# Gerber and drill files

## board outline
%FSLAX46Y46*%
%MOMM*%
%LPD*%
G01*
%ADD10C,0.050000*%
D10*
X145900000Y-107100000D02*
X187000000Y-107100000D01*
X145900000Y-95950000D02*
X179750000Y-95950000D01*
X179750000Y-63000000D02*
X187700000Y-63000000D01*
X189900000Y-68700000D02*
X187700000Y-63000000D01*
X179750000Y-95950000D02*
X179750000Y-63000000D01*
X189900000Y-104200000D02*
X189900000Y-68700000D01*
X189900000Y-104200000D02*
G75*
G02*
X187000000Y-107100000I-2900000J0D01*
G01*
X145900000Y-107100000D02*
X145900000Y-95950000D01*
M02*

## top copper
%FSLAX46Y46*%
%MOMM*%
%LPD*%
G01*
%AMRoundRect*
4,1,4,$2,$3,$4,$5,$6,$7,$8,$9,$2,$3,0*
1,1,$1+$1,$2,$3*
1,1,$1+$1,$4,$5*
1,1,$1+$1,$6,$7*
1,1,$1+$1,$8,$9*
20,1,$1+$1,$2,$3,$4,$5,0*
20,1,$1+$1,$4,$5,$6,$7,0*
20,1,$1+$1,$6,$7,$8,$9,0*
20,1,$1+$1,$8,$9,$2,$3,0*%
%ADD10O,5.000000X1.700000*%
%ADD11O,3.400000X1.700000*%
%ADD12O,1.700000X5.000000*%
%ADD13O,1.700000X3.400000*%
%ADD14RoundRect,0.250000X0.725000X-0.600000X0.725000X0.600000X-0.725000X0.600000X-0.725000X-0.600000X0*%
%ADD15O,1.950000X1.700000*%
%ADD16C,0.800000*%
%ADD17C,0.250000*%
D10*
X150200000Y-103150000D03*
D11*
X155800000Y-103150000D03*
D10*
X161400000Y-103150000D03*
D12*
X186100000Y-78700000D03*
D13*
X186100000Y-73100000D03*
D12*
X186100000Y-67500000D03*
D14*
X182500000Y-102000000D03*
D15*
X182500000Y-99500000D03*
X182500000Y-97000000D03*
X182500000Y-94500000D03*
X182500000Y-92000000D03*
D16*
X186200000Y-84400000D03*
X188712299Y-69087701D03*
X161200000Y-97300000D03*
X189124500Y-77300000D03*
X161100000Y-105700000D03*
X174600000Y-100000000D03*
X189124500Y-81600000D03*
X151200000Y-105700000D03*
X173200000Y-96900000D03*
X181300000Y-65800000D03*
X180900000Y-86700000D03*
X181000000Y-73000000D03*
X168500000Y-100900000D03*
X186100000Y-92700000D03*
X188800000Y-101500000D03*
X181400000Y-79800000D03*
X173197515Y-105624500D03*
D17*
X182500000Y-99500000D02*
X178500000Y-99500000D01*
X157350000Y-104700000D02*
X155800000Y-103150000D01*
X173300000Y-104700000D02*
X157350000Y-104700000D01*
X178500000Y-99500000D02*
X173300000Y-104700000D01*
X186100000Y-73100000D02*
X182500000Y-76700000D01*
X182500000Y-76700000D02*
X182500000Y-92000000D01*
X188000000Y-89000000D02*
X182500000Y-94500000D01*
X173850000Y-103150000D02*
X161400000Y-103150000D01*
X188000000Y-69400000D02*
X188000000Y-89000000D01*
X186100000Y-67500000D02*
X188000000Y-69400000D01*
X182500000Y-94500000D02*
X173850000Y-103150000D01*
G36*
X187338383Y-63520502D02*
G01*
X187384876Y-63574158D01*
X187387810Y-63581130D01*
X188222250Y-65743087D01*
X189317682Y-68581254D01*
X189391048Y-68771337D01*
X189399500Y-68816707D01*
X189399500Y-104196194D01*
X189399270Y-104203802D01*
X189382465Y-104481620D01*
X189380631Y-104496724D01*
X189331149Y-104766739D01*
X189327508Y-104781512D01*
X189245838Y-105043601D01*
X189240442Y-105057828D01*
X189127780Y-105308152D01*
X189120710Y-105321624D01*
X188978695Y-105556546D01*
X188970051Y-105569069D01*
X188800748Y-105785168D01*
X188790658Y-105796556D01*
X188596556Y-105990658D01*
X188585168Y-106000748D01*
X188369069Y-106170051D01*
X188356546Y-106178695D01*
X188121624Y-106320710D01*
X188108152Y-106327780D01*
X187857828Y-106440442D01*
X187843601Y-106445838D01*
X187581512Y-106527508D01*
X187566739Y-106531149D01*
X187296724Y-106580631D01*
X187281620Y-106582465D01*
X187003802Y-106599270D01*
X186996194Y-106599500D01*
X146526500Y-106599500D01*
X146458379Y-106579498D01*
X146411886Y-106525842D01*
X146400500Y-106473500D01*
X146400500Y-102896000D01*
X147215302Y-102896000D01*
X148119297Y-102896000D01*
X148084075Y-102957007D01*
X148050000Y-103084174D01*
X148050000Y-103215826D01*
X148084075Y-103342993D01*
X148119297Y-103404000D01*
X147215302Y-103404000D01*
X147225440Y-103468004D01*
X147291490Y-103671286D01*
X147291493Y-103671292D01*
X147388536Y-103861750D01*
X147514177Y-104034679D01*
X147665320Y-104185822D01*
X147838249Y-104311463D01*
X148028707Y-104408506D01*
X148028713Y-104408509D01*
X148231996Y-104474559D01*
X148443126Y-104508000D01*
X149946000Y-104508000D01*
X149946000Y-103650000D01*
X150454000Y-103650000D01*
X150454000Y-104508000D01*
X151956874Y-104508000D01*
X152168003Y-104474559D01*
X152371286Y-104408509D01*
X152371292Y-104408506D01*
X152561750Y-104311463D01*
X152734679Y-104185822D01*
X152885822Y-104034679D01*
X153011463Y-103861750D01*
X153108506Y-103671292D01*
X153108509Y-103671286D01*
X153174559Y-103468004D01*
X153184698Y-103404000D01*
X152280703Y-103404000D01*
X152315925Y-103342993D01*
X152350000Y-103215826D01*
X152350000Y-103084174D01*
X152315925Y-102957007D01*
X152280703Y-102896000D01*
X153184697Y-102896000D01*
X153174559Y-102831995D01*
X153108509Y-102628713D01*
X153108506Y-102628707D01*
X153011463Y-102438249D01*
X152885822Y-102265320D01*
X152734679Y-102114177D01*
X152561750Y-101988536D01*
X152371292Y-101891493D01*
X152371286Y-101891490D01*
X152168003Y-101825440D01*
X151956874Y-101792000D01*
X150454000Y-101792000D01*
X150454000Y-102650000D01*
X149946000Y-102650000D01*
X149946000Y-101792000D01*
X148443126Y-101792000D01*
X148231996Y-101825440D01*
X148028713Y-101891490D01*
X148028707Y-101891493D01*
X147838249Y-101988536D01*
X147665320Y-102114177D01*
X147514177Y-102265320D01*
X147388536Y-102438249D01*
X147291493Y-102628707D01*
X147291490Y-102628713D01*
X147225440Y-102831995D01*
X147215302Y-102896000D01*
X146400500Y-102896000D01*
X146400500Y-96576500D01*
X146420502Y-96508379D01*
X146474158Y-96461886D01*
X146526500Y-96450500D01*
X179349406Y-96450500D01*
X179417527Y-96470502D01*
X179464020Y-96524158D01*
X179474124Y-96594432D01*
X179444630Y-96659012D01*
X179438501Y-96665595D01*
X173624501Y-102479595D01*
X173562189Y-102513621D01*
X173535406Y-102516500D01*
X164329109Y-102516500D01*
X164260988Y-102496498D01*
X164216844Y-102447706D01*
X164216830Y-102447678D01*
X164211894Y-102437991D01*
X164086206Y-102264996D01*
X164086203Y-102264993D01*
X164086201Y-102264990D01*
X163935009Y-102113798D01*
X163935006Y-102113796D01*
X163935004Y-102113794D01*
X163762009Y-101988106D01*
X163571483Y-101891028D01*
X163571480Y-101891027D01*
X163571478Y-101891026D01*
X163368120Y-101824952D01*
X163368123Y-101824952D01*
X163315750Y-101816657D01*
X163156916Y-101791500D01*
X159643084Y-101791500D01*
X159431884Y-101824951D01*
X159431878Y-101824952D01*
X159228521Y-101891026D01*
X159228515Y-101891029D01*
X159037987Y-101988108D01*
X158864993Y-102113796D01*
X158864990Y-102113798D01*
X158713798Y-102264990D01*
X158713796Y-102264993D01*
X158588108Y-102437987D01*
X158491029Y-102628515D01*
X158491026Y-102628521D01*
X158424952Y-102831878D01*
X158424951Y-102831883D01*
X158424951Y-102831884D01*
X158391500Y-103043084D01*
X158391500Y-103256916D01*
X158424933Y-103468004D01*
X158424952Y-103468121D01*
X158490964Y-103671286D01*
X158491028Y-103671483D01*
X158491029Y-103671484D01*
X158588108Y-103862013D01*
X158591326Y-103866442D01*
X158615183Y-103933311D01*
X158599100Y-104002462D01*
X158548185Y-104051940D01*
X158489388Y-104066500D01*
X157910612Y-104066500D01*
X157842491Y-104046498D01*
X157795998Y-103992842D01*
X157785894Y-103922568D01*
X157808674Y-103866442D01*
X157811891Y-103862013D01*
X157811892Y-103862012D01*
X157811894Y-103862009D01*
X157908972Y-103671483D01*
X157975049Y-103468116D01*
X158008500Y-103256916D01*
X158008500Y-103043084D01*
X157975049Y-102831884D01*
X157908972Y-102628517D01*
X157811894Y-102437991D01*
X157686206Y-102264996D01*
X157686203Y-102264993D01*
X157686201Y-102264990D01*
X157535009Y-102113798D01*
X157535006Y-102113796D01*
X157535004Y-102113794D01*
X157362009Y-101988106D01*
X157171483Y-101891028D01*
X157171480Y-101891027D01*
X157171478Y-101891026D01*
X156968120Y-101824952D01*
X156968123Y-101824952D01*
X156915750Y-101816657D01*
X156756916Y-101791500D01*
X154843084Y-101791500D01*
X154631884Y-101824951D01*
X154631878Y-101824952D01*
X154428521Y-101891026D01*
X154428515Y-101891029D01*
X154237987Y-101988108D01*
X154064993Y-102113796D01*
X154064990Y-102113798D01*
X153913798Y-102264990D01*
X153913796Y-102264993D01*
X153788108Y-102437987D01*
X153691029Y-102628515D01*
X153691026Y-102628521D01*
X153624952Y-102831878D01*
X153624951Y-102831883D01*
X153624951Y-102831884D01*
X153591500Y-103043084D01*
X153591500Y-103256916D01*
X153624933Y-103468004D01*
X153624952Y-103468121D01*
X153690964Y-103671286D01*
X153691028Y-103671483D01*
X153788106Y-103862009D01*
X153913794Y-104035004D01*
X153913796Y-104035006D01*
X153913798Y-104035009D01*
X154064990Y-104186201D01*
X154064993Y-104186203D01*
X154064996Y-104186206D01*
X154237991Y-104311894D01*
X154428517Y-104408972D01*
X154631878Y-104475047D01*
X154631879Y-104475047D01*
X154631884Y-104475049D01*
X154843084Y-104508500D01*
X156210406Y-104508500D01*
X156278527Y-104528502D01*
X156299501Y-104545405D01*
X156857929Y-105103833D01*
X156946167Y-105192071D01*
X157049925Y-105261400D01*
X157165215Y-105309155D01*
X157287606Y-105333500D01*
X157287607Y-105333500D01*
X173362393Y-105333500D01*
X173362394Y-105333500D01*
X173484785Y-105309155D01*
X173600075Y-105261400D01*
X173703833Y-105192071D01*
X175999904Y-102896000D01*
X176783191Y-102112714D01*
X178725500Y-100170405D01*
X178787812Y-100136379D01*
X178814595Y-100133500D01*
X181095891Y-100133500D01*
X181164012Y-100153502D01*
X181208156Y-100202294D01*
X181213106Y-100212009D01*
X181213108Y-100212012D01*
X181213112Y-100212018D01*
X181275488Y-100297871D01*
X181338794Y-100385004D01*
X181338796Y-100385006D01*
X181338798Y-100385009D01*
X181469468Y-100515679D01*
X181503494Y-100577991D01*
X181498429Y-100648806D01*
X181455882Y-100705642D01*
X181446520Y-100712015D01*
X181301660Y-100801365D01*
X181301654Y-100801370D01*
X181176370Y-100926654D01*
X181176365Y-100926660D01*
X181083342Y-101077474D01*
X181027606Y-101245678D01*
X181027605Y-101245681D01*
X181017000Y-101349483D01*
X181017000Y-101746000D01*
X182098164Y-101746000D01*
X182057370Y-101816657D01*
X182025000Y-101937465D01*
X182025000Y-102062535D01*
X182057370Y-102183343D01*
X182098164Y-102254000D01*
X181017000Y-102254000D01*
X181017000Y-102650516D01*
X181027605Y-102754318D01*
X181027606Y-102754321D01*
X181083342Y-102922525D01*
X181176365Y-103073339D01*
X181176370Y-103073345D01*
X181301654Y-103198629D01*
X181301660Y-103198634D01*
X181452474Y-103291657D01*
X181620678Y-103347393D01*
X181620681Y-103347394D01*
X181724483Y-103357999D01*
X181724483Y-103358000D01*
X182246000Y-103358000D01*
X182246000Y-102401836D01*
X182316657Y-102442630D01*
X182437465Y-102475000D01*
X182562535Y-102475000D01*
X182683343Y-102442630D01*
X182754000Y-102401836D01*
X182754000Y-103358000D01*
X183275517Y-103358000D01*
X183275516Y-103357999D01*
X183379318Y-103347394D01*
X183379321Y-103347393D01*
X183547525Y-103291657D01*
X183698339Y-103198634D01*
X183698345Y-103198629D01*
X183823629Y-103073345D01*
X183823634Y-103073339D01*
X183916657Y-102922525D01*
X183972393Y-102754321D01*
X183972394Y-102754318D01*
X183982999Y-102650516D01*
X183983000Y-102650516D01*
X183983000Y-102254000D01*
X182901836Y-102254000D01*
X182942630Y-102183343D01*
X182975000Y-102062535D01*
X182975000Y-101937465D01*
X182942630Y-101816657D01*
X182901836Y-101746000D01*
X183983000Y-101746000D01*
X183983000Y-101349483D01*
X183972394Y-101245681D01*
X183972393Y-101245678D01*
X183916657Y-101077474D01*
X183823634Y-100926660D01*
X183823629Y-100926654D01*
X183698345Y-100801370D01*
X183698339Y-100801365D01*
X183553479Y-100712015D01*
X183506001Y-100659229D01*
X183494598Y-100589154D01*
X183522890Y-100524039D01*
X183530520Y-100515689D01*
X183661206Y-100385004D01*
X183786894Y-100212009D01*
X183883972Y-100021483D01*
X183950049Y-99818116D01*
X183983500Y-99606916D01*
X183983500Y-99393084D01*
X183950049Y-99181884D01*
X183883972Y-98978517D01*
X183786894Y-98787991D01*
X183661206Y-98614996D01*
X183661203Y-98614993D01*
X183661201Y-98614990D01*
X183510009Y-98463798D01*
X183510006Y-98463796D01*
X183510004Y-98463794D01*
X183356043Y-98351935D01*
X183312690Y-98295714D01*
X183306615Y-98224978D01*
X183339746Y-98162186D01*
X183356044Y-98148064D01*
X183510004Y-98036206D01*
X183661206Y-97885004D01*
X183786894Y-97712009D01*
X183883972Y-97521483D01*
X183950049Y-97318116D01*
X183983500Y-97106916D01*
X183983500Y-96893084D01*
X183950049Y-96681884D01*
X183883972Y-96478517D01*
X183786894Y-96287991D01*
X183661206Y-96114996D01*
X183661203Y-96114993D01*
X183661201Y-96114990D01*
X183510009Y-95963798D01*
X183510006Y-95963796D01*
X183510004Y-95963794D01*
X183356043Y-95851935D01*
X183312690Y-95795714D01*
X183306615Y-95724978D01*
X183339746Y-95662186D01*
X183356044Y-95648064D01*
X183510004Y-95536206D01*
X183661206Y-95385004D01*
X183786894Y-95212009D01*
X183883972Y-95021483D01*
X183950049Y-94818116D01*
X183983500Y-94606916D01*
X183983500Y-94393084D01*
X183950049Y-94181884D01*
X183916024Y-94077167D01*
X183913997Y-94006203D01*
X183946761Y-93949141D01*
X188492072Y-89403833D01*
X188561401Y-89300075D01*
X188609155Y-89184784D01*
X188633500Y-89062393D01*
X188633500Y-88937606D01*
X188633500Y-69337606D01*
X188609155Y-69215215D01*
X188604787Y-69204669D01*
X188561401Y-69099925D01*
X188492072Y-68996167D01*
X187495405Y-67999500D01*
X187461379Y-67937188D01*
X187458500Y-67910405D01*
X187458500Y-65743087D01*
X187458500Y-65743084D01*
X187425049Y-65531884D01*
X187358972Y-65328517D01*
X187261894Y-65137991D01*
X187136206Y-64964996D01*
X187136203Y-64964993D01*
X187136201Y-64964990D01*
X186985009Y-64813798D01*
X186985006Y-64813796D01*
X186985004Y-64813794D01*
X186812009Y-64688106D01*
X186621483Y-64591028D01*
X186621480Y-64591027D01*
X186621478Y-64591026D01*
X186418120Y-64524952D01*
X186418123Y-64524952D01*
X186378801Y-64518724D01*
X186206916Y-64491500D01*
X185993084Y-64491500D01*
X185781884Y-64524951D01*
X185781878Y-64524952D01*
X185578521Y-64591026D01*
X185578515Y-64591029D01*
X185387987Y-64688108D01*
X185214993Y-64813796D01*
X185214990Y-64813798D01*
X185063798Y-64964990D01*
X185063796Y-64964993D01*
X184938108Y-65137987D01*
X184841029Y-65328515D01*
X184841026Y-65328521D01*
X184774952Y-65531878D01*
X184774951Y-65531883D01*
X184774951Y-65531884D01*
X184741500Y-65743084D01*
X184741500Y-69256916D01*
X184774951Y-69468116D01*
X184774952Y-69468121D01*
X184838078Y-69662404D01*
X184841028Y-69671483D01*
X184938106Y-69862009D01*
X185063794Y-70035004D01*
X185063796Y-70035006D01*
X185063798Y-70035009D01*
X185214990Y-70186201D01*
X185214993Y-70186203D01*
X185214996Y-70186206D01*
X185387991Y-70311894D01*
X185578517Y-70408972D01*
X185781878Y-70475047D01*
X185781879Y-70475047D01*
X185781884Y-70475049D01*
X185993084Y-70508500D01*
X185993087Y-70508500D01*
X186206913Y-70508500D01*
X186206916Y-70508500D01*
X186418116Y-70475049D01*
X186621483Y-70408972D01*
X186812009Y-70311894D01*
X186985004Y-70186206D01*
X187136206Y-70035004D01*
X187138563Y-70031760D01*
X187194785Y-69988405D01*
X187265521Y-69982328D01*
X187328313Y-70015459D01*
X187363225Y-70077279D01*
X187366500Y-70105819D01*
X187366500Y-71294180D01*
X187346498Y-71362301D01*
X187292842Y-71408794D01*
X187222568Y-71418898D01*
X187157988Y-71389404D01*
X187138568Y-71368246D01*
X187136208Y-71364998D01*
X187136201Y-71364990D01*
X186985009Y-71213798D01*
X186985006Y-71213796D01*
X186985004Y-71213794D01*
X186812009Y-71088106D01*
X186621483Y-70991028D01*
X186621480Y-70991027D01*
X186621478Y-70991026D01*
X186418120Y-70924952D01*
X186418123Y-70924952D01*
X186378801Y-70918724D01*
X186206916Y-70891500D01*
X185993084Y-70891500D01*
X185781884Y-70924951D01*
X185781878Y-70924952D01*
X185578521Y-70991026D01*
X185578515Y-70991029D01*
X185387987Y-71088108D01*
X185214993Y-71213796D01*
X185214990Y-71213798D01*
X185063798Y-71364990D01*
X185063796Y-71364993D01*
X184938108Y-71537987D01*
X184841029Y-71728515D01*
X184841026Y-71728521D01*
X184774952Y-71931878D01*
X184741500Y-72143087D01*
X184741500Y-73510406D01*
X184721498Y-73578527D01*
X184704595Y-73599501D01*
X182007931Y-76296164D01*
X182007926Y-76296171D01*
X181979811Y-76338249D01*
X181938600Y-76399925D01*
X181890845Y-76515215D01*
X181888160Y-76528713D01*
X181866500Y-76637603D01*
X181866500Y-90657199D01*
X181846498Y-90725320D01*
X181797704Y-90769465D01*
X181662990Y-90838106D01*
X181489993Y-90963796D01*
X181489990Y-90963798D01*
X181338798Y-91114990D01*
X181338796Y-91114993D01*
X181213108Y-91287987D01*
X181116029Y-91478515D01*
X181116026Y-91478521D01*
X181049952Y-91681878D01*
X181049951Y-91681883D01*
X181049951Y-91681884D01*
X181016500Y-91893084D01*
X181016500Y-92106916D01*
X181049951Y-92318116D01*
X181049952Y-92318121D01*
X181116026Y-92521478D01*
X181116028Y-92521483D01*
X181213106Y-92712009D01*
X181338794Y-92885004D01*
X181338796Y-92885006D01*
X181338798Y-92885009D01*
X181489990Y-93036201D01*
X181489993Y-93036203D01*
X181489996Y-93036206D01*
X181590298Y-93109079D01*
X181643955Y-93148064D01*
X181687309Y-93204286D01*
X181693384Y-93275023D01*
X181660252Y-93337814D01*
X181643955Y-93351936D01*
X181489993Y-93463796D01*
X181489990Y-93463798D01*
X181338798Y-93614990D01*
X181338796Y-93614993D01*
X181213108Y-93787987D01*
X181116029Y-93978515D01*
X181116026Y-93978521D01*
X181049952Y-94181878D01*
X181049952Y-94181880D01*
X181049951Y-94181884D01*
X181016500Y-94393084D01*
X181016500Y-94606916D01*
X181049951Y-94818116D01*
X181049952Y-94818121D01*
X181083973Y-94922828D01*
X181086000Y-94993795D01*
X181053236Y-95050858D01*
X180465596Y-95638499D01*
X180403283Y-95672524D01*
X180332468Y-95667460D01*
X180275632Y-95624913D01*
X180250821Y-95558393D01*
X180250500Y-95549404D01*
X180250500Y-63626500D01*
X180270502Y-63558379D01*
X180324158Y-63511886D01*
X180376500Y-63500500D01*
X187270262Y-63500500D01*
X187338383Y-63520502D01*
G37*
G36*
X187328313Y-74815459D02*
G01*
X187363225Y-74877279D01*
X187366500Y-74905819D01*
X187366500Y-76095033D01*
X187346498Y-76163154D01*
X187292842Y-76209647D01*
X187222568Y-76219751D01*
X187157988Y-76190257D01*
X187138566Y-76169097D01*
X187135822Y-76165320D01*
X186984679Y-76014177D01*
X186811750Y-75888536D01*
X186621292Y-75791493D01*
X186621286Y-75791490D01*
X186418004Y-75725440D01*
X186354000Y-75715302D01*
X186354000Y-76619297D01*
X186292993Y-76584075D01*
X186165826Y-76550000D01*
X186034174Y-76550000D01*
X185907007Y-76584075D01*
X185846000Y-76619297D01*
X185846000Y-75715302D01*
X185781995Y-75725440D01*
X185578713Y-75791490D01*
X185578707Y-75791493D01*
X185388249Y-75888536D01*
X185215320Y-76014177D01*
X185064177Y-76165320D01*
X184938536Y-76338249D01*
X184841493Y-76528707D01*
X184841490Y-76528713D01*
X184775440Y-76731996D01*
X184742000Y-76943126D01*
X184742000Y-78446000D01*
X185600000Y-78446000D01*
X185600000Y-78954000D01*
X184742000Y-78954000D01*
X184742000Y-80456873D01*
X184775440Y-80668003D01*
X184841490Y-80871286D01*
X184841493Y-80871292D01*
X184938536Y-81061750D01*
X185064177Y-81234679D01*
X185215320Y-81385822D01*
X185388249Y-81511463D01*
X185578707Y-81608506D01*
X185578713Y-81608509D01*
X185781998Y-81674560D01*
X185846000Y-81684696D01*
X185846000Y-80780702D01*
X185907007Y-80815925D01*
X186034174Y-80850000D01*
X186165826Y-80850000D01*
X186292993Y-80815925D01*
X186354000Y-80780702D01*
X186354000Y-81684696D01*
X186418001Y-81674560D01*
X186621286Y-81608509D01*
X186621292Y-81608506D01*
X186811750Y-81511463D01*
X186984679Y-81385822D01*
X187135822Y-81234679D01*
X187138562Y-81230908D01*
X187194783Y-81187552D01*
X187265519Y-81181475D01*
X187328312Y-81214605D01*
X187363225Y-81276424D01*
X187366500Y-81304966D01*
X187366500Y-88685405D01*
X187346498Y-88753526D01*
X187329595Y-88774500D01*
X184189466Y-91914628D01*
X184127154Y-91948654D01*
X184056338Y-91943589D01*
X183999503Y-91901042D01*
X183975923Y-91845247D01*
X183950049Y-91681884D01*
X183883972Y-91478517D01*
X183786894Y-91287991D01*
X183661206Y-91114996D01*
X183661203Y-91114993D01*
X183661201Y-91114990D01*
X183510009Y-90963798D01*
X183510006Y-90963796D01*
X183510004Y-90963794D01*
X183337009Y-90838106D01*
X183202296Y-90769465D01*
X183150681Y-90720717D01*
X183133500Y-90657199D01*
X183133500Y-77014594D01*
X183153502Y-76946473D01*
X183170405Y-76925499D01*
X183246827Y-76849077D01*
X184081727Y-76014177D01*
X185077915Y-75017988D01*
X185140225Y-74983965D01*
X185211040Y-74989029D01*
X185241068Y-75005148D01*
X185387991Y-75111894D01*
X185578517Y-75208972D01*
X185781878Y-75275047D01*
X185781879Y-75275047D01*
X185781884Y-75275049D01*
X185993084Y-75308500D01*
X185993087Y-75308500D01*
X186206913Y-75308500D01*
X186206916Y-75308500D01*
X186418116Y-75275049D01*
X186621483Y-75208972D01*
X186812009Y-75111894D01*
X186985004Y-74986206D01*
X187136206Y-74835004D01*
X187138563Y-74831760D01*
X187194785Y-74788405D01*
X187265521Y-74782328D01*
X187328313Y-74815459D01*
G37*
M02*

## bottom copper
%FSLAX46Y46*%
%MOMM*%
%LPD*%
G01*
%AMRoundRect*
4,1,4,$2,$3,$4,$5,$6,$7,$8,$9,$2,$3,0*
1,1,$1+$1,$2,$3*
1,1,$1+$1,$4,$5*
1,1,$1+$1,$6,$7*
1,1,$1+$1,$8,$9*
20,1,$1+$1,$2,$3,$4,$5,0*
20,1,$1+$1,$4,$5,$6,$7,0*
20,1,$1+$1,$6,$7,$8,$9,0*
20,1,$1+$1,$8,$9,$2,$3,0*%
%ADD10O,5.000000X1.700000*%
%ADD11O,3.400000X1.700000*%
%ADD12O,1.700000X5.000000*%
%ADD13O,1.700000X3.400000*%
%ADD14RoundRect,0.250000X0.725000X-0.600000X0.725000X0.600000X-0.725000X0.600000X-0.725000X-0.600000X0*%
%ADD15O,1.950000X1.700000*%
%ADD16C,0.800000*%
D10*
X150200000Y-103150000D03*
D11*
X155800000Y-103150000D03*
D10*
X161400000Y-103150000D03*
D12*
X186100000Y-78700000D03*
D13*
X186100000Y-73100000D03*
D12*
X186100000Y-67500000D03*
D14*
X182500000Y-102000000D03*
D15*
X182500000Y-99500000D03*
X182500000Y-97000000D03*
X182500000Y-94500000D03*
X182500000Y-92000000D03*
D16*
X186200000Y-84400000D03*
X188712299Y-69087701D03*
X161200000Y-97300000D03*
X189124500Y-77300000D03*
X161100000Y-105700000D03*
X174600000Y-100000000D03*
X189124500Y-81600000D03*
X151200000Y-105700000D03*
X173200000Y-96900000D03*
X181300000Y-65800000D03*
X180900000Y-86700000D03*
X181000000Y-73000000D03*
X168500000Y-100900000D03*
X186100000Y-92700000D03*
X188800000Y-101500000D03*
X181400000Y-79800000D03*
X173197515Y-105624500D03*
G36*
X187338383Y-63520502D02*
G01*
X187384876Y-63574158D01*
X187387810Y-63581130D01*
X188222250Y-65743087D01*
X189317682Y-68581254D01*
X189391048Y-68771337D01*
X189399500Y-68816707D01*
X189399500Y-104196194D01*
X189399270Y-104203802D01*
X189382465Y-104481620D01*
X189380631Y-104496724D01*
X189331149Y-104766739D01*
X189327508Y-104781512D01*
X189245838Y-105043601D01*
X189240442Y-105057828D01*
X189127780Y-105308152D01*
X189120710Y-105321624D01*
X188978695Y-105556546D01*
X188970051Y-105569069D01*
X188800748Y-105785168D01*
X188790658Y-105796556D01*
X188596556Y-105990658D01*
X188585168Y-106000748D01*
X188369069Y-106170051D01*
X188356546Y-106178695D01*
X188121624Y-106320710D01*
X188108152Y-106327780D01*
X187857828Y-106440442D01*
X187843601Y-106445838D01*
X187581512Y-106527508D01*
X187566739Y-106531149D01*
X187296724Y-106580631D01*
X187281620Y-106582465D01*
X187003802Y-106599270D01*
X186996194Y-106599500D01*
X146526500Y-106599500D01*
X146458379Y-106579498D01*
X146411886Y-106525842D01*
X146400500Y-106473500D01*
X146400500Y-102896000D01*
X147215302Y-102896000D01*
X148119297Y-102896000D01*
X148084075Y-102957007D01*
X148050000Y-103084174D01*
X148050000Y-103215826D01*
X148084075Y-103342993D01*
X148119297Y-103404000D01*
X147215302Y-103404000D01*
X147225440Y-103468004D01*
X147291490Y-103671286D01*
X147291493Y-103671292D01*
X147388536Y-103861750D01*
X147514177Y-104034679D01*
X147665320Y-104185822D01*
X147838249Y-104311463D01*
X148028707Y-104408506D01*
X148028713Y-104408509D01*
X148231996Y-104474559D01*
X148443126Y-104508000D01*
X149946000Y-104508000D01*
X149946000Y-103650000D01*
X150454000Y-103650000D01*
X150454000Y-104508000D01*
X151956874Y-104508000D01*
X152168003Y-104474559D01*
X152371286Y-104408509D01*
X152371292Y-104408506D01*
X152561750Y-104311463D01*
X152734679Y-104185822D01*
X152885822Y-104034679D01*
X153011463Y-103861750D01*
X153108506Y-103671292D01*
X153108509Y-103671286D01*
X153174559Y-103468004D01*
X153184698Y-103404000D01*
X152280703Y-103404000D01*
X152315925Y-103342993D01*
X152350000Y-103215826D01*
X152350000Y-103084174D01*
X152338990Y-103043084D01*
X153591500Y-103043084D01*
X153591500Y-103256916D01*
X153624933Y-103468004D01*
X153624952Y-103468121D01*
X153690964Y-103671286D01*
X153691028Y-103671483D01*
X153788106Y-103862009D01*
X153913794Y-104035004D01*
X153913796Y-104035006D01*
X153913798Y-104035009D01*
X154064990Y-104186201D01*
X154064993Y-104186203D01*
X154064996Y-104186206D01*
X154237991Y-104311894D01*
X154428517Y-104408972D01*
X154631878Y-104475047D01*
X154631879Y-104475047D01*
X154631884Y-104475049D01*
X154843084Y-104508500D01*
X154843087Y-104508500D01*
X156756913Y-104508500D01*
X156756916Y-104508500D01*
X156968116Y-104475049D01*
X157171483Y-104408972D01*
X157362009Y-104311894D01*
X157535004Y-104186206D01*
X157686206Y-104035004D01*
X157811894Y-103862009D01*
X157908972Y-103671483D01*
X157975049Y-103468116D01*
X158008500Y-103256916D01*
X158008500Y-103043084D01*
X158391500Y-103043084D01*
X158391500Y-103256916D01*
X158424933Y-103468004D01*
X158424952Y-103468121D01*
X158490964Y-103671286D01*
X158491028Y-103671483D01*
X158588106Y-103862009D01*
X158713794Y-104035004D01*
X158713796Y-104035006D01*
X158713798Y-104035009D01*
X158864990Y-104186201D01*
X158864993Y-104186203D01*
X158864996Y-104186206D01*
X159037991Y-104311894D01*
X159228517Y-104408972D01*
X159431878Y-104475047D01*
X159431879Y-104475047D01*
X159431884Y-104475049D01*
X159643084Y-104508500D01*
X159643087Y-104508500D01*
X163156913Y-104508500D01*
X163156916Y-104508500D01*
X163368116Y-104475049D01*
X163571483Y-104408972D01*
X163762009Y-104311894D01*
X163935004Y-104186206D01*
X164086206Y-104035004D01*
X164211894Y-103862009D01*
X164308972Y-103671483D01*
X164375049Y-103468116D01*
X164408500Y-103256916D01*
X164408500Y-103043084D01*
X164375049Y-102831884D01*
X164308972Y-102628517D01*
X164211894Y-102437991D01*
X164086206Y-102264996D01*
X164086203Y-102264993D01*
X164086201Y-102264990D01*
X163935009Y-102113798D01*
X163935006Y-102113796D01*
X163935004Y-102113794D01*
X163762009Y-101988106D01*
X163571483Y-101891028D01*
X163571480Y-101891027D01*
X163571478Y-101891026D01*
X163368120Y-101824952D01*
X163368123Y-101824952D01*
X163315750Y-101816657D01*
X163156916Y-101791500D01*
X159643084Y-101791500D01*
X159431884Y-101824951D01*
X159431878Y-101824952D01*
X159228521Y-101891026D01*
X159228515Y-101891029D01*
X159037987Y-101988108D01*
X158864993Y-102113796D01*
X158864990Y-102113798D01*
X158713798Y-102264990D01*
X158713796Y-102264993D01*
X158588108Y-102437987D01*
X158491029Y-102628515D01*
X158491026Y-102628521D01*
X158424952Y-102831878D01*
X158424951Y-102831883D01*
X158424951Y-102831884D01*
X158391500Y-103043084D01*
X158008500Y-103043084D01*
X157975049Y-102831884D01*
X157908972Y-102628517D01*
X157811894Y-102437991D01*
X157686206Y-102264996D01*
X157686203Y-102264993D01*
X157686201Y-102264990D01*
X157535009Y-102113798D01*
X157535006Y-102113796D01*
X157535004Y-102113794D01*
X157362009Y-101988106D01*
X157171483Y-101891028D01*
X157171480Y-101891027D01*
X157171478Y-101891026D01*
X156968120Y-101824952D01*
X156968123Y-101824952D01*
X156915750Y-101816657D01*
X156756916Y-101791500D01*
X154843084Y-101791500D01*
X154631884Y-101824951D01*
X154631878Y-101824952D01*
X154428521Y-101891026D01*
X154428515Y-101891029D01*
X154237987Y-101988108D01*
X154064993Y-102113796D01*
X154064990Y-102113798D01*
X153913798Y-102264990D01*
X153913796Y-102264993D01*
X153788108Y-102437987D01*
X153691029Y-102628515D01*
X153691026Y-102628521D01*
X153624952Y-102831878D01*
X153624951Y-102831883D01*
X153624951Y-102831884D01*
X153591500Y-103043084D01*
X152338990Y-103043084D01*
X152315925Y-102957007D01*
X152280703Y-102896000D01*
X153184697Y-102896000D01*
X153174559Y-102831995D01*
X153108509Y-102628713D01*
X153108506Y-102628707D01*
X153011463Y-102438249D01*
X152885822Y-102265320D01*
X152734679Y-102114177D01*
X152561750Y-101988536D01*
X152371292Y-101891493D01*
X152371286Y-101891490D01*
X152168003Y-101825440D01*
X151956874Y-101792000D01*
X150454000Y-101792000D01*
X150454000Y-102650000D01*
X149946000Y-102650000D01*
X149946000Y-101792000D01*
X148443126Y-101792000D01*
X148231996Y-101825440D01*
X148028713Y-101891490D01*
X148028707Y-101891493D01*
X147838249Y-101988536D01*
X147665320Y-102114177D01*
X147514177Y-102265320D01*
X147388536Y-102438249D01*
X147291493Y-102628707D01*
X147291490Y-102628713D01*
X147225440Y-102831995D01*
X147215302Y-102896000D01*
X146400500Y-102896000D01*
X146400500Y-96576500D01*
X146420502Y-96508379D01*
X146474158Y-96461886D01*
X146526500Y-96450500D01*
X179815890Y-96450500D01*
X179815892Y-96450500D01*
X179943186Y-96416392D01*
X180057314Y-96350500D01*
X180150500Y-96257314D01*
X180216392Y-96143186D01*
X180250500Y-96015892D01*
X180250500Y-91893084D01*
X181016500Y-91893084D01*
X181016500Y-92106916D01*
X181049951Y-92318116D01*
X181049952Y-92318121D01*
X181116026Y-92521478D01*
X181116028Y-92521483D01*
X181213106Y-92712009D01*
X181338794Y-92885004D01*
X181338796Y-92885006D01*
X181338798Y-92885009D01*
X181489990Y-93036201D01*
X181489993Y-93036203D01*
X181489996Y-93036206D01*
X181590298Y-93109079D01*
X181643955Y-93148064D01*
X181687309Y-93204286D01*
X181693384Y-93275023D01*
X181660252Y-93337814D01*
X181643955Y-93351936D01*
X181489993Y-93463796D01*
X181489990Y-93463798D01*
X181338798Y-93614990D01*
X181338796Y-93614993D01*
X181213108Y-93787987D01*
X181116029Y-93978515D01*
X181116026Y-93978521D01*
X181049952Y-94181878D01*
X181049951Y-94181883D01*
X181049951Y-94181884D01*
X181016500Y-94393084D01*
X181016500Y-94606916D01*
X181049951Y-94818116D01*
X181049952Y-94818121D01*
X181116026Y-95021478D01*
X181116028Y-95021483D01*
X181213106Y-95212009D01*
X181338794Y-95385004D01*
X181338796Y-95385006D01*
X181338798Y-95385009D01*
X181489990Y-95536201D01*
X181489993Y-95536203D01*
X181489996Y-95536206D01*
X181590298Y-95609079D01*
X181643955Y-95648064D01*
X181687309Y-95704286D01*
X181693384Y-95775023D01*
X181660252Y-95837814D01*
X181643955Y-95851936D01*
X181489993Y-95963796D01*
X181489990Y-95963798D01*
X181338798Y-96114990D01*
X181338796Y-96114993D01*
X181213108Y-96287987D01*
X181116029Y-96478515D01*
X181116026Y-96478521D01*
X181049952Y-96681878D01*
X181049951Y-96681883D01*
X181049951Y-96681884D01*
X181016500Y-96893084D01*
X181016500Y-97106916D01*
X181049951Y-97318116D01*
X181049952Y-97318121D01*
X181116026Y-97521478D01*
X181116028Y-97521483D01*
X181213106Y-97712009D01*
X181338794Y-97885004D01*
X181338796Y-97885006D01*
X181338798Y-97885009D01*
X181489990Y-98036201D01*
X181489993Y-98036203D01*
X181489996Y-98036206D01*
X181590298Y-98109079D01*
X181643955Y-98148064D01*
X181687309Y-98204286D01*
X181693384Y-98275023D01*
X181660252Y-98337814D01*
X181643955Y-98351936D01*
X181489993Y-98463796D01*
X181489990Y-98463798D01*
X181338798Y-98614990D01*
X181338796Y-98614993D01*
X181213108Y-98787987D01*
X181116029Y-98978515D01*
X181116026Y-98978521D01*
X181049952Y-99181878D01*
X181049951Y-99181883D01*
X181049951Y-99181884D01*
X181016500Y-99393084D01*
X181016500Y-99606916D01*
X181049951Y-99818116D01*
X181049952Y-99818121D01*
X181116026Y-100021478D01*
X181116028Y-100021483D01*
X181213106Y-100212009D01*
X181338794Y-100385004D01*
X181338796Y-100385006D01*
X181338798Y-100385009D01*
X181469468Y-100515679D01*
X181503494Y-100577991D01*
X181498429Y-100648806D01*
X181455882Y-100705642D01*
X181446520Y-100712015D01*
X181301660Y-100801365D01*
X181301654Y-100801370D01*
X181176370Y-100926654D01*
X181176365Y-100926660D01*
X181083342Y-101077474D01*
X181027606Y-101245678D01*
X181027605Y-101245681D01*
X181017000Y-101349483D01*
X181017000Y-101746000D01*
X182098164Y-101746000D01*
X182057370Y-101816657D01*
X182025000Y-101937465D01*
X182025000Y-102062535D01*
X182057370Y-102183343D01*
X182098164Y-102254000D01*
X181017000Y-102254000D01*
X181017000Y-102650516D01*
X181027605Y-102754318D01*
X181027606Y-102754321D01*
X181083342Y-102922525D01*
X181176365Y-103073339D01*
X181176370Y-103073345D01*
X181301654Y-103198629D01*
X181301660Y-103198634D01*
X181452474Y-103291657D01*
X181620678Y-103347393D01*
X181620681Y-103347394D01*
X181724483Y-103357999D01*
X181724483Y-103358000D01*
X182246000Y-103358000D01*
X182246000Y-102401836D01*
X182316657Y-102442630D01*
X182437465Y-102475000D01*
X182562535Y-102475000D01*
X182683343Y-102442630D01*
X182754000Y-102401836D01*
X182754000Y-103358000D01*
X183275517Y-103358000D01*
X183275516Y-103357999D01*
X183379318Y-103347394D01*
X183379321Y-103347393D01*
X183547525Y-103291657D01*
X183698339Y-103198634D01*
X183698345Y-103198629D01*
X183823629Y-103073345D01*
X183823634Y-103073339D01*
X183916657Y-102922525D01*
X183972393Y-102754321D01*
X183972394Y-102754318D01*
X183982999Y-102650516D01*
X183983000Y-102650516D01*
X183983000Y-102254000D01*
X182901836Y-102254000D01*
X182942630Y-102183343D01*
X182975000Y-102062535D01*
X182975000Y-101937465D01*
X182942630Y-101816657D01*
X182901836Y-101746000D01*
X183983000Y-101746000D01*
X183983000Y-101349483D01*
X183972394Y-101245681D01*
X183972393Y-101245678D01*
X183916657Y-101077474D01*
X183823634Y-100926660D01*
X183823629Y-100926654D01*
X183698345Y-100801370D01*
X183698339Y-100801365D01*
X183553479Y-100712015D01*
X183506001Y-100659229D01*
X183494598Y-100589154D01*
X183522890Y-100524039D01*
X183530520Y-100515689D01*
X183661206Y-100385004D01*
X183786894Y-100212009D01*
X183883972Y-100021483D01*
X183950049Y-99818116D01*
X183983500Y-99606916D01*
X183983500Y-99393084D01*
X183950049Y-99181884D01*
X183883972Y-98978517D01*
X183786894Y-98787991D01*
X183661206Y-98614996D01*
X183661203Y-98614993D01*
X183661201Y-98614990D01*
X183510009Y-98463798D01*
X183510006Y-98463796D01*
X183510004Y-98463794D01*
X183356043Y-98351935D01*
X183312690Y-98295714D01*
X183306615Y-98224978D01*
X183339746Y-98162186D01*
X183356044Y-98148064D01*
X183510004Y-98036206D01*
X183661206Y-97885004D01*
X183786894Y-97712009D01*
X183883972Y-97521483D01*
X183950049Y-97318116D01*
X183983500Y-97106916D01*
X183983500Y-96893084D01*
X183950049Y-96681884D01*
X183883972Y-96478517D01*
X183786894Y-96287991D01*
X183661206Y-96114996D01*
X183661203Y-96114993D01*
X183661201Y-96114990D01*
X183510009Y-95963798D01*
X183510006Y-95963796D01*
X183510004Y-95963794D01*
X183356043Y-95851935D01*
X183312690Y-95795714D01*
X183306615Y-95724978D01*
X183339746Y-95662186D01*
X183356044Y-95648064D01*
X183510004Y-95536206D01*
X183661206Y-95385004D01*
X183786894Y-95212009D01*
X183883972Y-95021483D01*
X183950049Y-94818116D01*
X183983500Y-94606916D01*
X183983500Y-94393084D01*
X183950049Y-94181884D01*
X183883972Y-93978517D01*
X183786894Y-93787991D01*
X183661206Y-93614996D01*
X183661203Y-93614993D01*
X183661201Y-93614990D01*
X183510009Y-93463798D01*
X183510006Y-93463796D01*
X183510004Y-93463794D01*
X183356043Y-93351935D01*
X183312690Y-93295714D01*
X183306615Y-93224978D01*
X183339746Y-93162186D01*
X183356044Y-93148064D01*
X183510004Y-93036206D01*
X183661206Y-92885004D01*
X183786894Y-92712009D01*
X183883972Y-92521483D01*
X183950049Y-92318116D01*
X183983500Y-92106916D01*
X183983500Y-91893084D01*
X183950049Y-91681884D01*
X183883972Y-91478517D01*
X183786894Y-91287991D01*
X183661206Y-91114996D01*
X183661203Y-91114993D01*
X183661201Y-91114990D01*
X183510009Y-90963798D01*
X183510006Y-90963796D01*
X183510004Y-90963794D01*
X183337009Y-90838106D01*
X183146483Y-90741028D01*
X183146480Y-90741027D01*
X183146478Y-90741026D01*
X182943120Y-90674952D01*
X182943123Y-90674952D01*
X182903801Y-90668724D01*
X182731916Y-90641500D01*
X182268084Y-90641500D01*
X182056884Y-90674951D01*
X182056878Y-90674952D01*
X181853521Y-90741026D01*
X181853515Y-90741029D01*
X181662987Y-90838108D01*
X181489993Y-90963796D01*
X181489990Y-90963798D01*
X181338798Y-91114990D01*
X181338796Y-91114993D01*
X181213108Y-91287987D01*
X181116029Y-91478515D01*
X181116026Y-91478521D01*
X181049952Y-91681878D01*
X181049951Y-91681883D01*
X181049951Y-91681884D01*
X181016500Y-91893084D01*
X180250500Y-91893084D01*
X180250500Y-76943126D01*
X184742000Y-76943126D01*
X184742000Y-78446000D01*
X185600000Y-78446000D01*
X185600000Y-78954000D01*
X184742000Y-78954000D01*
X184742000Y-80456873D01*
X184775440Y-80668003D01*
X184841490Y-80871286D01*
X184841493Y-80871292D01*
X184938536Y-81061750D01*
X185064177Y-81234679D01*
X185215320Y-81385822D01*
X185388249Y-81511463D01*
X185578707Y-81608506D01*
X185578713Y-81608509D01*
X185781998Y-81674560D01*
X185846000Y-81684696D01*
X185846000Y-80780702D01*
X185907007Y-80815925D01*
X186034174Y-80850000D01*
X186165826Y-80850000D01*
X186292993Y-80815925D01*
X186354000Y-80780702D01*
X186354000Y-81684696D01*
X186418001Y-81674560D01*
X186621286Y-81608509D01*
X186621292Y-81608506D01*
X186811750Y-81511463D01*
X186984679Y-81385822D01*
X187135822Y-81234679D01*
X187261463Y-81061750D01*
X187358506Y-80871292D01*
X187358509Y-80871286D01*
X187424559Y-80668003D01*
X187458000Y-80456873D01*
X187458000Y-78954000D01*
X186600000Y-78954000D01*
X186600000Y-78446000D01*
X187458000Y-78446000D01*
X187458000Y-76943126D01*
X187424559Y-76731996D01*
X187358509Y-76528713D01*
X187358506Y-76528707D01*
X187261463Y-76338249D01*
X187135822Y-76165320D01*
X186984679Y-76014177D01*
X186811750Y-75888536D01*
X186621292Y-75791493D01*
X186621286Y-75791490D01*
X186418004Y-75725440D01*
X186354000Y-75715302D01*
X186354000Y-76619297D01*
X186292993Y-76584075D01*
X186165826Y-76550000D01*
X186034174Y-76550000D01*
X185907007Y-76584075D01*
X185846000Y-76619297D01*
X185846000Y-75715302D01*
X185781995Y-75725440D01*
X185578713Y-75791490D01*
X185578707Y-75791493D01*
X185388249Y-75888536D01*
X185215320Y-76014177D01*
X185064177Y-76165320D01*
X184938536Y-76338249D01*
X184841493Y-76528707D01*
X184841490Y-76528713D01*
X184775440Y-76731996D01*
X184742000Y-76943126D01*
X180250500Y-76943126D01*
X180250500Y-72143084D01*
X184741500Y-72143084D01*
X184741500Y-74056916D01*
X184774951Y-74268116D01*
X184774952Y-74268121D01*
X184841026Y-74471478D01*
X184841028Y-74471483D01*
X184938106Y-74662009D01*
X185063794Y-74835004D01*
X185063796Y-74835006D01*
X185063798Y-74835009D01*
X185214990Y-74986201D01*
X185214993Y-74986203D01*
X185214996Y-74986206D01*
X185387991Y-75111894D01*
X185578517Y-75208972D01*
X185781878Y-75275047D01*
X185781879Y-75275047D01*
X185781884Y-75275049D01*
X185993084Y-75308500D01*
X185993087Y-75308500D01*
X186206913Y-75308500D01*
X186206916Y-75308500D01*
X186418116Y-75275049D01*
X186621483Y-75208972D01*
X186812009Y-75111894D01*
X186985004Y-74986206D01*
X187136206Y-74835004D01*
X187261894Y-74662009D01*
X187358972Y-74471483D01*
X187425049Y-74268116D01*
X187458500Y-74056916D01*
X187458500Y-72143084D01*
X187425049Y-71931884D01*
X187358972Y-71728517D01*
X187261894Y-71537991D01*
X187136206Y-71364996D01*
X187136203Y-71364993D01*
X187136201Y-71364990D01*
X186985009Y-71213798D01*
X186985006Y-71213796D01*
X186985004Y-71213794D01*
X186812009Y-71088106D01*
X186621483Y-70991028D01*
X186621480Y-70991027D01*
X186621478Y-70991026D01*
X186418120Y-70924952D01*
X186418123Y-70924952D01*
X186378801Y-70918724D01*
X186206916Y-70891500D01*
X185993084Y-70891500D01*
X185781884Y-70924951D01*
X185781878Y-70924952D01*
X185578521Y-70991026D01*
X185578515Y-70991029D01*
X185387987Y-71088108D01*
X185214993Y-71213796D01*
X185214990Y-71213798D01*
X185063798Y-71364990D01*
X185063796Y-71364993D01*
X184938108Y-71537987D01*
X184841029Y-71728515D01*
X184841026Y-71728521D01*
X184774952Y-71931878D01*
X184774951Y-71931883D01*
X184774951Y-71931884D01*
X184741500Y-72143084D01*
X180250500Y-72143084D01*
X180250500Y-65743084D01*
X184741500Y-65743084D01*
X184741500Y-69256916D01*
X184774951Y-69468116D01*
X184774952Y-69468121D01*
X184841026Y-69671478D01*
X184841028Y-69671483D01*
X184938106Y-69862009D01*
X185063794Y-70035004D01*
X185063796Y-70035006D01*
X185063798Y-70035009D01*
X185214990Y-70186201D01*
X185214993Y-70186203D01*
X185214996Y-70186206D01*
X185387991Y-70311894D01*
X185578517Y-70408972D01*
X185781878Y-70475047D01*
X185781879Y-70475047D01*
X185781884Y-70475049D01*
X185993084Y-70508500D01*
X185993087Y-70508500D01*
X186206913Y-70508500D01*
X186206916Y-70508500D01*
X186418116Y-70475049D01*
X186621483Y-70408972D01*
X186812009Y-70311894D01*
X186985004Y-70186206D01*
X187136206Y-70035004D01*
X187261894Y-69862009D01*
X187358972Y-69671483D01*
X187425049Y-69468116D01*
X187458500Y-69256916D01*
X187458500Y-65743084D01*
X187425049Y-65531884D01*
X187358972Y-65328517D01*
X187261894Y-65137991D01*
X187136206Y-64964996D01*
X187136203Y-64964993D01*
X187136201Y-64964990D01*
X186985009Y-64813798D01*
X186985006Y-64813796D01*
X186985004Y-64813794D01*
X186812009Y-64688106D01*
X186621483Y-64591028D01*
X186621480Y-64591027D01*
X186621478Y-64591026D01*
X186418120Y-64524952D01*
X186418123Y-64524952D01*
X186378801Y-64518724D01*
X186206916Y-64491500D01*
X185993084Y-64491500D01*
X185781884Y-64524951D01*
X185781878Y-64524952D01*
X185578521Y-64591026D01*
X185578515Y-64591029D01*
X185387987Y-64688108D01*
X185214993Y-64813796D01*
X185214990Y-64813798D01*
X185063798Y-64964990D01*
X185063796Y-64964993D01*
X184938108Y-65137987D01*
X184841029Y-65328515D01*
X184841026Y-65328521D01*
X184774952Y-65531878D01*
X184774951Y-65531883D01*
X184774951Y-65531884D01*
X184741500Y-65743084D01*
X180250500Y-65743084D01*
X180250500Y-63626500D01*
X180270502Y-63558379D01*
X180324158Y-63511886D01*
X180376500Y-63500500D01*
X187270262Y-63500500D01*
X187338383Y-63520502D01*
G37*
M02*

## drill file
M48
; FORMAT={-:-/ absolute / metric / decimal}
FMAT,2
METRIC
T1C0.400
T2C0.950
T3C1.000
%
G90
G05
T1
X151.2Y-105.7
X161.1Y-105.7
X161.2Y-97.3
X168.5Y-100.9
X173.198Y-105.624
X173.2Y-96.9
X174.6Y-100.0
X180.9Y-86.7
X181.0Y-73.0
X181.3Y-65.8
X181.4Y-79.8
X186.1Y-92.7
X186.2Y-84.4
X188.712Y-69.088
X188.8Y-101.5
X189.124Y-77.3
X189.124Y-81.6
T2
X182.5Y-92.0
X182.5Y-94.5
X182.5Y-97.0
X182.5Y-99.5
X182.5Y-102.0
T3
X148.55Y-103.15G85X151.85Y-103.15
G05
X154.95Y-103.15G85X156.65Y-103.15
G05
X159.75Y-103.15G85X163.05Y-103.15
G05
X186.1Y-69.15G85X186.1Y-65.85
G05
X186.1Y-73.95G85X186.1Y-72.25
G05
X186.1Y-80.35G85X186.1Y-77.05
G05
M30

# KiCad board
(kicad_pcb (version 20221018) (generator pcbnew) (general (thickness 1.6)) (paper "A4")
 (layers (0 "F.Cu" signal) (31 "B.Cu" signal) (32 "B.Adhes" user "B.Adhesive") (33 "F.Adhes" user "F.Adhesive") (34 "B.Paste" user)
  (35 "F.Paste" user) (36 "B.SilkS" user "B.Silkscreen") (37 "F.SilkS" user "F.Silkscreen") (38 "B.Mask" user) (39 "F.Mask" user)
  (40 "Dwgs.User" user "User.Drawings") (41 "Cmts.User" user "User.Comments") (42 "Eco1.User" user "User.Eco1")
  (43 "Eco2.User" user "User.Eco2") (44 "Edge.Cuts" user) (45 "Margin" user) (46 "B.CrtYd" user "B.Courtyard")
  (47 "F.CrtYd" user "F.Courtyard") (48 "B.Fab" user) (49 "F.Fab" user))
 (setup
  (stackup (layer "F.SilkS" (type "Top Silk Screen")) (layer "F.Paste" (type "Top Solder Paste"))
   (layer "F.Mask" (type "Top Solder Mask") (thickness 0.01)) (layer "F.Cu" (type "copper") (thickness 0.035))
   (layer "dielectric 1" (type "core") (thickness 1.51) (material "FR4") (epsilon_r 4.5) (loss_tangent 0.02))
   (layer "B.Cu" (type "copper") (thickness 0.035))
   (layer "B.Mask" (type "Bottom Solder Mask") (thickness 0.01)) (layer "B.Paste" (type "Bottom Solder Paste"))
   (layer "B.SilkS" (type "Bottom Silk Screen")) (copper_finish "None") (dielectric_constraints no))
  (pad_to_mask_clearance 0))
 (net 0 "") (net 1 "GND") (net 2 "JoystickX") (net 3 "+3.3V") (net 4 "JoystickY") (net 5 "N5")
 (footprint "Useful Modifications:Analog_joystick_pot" (layer "F.Cu") (at 155.8 103.15 90)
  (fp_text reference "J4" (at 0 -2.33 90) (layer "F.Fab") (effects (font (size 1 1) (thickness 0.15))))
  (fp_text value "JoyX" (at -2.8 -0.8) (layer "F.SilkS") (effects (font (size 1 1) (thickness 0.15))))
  (pad "1" thru_hole oval (at 0 -5.6 90) (size 1.7 5) (drill oval 1 4.3) (layers "*.Cu" "*.Mask") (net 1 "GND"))
  (pad "2" thru_hole oval (at 0 0 90) (size 1.7 3.4) (drill oval 1 2.7) (layers "*.Cu" "*.Mask") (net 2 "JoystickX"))
  (pad "3" thru_hole oval (at 0 5.6 90) (size 1.7 5) (drill oval 1 4.3) (layers "*.Cu" "*.Mask") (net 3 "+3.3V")))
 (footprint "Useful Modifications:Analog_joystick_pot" (layer "F.Cu") (at 186.1 73.1 180)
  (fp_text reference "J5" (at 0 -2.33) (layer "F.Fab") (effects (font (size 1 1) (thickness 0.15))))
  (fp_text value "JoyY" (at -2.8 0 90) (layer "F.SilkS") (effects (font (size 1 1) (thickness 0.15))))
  (pad "1" thru_hole oval (at 0 -5.6 180) (size 1.7 5) (drill oval 1 4.3) (layers "*.Cu" "*.Mask") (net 1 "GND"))
  (pad "2" thru_hole oval (at 0 0 180) (size 1.7 3.4) (drill oval 1 2.7) (layers "*.Cu" "*.Mask") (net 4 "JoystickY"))
  (pad "3" thru_hole oval (at 0 5.6 180) (size 1.7 5) (drill oval 1 4.3) (layers "*.Cu" "*.Mask") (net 3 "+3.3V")))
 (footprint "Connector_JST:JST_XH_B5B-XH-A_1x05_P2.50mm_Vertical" (layer "F.Cu") (at 182.5 102 90)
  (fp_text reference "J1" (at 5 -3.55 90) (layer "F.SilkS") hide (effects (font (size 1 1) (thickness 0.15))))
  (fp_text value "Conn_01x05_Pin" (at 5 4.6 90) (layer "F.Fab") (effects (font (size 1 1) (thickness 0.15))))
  (pad "1" thru_hole roundrect (at 0 0 90) (size 1.7 1.95) (drill 0.95) (layers "*.Cu" "*.Mask") (roundrect_rratio 0.1470588235)
   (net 1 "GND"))
  (pad "2" thru_hole oval (at 2.5 0 90) (size 1.7 1.95) (drill 0.95) (layers "*.Cu" "*.Mask") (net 2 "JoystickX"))
  (pad "3" thru_hole oval (at 5 0 90) (size 1.7 1.95) (drill 0.95) (layers "*.Cu" "*.Mask") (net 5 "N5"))
  (pad "4" thru_hole oval (at 7.5 0 90) (size 1.7 1.95) (drill 0.95) (layers "*.Cu" "*.Mask") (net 3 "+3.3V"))
  (pad "5" thru_hole oval (at 10 0 90) (size 1.7 1.95) (drill 0.95) (layers "*.Cu" "*.Mask") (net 4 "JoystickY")))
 (gr_line (start 145.9 107.1) (end 187 107.1) (stroke (width 0.05) (type default)) (layer "Edge.Cuts"))
 (gr_line (start 145.9 95.95) (end 179.75 95.95) (stroke (width 0.05) (type default)) (layer "Edge.Cuts"))
 (gr_line (start 179.75 63) (end 187.7 63) (stroke (width 0.05) (type default)) (layer "Edge.Cuts"))
 (gr_line (start 189.9 68.7) (end 187.7 63) (stroke (width 0.05) (type default)) (layer "Edge.Cuts"))
 (gr_line (start 179.75 95.95) (end 179.75 63) (stroke (width 0.05) (type default)) (layer "Edge.Cuts"))
 (gr_line (start 189.9 104.2) (end 189.9 68.7) (stroke (width 0.05) (type default)) (layer "Edge.Cuts"))
 (gr_arc (start 189.9 104.2) (mid 189.05061 106.25061) (end 187 107.1) (stroke (width 0.05) (type default)) (layer "Edge.Cuts"))
 (gr_line (start 145.9 107.1) (end 145.9 95.95) (stroke (width 0.05) (type default)) (layer "Edge.Cuts"))
 (via (at 186.2 84.4) (size 0.8) (drill 0.4) (layers "F.Cu" "B.Cu") (free) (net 1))
 (via (at 188.712299 69.087701) (size 0.8) (drill 0.4) (layers "F.Cu" "B.Cu") (free) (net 1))
 (via (at 161.2 97.3) (size 0.8) (drill 0.4) (layers "F.Cu" "B.Cu") (free) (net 1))
 (via (at 189.1245 77.3) (size 0.8) (drill 0.4) (layers "F.Cu" "B.Cu") (free) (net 1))
 (via (at 161.1 105.7) (size 0.8) (drill 0.4) (layers "F.Cu" "B.Cu") (free) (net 1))
 (via (at 174.6 100) (size 0.8) (drill 0.4) (layers "F.Cu" "B.Cu") (free) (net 1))
 (via (at 189.1245 81.6) (size 0.8) (drill 0.4) (layers "F.Cu" "B.Cu") (free) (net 1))
 (via (at 151.2 105.7) (size 0.8) (drill 0.4) (layers "F.Cu" "B.Cu") (free) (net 1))
 (via (at 173.2 96.9) (size 0.8) (drill 0.4) (layers "F.Cu" "B.Cu") (free) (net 1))
 (via (at 181.3 65.8) (size 0.8) (drill 0.4) (layers "F.Cu" "B.Cu") (free) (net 1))
 (via (at 180.9 86.7) (size 0.8) (drill 0.4) (layers "F.Cu" "B.Cu") (free) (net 1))
 (via (at 181 73) (size 0.8) (drill 0.4) (layers "F.Cu" "B.Cu") (free) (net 1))
 (via (at 168.5 100.9) (size 0.8) (drill 0.4) (layers "F.Cu" "B.Cu") (free) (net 1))
 (via (at 186.1 92.7) (size 0.8) (drill 0.4) (layers "F.Cu" "B.Cu") (free) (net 1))
 (via (at 188.8 101.5) (size 0.8) (drill 0.4) (layers "F.Cu" "B.Cu") (free) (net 1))
 (via (at 181.4 79.8) (size 0.8) (drill 0.4) (layers "F.Cu" "B.Cu") (free) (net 1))
 (via (at 173.197515 105.6245) (size 0.8) (drill 0.4) (layers "F.Cu" "B.Cu") (free) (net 1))
 (segment (start 182.5 99.5) (end 178.5 99.5) (width 0.25) (layer "F.Cu") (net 2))
 (segment (start 157.35 104.7) (end 155.8 103.15) (width 0.25) (layer "F.Cu") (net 2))
 (segment (start 173.3 104.7) (end 157.35 104.7) (width 0.25) (layer "F.Cu") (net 2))
 (segment (start 178.5 99.5) (end 173.3 104.7) (width 0.25) (layer "F.Cu") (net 2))
 (segment (start 186.1 73.1) (end 182.5 76.7) (width 0.25) (layer "F.Cu") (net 4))
 (segment (start 182.5 76.7) (end 182.5 92) (width 0.25) (layer "F.Cu") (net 4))
 (segment (start 188 89) (end 182.5 94.5) (width 0.25) (layer "F.Cu") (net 3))
 (segment (start 173.85 103.15) (end 161.4 103.15) (width 0.25) (layer "F.Cu") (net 3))
 (segment (start 188 69.4) (end 188 89) (width 0.25) (layer "F.Cu") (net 3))
 (segment (start 186.1 67.5) (end 188 69.4) (width 0.25) (layer "F.Cu") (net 3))
 (segment (start 182.5 94.5) (end 173.85 103.15) (width 0.25) (layer "F.Cu") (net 3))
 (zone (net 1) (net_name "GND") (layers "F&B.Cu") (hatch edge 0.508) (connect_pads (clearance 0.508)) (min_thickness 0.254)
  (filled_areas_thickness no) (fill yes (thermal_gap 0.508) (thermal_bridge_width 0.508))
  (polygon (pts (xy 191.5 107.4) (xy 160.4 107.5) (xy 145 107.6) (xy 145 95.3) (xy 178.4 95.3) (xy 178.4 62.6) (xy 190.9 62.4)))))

